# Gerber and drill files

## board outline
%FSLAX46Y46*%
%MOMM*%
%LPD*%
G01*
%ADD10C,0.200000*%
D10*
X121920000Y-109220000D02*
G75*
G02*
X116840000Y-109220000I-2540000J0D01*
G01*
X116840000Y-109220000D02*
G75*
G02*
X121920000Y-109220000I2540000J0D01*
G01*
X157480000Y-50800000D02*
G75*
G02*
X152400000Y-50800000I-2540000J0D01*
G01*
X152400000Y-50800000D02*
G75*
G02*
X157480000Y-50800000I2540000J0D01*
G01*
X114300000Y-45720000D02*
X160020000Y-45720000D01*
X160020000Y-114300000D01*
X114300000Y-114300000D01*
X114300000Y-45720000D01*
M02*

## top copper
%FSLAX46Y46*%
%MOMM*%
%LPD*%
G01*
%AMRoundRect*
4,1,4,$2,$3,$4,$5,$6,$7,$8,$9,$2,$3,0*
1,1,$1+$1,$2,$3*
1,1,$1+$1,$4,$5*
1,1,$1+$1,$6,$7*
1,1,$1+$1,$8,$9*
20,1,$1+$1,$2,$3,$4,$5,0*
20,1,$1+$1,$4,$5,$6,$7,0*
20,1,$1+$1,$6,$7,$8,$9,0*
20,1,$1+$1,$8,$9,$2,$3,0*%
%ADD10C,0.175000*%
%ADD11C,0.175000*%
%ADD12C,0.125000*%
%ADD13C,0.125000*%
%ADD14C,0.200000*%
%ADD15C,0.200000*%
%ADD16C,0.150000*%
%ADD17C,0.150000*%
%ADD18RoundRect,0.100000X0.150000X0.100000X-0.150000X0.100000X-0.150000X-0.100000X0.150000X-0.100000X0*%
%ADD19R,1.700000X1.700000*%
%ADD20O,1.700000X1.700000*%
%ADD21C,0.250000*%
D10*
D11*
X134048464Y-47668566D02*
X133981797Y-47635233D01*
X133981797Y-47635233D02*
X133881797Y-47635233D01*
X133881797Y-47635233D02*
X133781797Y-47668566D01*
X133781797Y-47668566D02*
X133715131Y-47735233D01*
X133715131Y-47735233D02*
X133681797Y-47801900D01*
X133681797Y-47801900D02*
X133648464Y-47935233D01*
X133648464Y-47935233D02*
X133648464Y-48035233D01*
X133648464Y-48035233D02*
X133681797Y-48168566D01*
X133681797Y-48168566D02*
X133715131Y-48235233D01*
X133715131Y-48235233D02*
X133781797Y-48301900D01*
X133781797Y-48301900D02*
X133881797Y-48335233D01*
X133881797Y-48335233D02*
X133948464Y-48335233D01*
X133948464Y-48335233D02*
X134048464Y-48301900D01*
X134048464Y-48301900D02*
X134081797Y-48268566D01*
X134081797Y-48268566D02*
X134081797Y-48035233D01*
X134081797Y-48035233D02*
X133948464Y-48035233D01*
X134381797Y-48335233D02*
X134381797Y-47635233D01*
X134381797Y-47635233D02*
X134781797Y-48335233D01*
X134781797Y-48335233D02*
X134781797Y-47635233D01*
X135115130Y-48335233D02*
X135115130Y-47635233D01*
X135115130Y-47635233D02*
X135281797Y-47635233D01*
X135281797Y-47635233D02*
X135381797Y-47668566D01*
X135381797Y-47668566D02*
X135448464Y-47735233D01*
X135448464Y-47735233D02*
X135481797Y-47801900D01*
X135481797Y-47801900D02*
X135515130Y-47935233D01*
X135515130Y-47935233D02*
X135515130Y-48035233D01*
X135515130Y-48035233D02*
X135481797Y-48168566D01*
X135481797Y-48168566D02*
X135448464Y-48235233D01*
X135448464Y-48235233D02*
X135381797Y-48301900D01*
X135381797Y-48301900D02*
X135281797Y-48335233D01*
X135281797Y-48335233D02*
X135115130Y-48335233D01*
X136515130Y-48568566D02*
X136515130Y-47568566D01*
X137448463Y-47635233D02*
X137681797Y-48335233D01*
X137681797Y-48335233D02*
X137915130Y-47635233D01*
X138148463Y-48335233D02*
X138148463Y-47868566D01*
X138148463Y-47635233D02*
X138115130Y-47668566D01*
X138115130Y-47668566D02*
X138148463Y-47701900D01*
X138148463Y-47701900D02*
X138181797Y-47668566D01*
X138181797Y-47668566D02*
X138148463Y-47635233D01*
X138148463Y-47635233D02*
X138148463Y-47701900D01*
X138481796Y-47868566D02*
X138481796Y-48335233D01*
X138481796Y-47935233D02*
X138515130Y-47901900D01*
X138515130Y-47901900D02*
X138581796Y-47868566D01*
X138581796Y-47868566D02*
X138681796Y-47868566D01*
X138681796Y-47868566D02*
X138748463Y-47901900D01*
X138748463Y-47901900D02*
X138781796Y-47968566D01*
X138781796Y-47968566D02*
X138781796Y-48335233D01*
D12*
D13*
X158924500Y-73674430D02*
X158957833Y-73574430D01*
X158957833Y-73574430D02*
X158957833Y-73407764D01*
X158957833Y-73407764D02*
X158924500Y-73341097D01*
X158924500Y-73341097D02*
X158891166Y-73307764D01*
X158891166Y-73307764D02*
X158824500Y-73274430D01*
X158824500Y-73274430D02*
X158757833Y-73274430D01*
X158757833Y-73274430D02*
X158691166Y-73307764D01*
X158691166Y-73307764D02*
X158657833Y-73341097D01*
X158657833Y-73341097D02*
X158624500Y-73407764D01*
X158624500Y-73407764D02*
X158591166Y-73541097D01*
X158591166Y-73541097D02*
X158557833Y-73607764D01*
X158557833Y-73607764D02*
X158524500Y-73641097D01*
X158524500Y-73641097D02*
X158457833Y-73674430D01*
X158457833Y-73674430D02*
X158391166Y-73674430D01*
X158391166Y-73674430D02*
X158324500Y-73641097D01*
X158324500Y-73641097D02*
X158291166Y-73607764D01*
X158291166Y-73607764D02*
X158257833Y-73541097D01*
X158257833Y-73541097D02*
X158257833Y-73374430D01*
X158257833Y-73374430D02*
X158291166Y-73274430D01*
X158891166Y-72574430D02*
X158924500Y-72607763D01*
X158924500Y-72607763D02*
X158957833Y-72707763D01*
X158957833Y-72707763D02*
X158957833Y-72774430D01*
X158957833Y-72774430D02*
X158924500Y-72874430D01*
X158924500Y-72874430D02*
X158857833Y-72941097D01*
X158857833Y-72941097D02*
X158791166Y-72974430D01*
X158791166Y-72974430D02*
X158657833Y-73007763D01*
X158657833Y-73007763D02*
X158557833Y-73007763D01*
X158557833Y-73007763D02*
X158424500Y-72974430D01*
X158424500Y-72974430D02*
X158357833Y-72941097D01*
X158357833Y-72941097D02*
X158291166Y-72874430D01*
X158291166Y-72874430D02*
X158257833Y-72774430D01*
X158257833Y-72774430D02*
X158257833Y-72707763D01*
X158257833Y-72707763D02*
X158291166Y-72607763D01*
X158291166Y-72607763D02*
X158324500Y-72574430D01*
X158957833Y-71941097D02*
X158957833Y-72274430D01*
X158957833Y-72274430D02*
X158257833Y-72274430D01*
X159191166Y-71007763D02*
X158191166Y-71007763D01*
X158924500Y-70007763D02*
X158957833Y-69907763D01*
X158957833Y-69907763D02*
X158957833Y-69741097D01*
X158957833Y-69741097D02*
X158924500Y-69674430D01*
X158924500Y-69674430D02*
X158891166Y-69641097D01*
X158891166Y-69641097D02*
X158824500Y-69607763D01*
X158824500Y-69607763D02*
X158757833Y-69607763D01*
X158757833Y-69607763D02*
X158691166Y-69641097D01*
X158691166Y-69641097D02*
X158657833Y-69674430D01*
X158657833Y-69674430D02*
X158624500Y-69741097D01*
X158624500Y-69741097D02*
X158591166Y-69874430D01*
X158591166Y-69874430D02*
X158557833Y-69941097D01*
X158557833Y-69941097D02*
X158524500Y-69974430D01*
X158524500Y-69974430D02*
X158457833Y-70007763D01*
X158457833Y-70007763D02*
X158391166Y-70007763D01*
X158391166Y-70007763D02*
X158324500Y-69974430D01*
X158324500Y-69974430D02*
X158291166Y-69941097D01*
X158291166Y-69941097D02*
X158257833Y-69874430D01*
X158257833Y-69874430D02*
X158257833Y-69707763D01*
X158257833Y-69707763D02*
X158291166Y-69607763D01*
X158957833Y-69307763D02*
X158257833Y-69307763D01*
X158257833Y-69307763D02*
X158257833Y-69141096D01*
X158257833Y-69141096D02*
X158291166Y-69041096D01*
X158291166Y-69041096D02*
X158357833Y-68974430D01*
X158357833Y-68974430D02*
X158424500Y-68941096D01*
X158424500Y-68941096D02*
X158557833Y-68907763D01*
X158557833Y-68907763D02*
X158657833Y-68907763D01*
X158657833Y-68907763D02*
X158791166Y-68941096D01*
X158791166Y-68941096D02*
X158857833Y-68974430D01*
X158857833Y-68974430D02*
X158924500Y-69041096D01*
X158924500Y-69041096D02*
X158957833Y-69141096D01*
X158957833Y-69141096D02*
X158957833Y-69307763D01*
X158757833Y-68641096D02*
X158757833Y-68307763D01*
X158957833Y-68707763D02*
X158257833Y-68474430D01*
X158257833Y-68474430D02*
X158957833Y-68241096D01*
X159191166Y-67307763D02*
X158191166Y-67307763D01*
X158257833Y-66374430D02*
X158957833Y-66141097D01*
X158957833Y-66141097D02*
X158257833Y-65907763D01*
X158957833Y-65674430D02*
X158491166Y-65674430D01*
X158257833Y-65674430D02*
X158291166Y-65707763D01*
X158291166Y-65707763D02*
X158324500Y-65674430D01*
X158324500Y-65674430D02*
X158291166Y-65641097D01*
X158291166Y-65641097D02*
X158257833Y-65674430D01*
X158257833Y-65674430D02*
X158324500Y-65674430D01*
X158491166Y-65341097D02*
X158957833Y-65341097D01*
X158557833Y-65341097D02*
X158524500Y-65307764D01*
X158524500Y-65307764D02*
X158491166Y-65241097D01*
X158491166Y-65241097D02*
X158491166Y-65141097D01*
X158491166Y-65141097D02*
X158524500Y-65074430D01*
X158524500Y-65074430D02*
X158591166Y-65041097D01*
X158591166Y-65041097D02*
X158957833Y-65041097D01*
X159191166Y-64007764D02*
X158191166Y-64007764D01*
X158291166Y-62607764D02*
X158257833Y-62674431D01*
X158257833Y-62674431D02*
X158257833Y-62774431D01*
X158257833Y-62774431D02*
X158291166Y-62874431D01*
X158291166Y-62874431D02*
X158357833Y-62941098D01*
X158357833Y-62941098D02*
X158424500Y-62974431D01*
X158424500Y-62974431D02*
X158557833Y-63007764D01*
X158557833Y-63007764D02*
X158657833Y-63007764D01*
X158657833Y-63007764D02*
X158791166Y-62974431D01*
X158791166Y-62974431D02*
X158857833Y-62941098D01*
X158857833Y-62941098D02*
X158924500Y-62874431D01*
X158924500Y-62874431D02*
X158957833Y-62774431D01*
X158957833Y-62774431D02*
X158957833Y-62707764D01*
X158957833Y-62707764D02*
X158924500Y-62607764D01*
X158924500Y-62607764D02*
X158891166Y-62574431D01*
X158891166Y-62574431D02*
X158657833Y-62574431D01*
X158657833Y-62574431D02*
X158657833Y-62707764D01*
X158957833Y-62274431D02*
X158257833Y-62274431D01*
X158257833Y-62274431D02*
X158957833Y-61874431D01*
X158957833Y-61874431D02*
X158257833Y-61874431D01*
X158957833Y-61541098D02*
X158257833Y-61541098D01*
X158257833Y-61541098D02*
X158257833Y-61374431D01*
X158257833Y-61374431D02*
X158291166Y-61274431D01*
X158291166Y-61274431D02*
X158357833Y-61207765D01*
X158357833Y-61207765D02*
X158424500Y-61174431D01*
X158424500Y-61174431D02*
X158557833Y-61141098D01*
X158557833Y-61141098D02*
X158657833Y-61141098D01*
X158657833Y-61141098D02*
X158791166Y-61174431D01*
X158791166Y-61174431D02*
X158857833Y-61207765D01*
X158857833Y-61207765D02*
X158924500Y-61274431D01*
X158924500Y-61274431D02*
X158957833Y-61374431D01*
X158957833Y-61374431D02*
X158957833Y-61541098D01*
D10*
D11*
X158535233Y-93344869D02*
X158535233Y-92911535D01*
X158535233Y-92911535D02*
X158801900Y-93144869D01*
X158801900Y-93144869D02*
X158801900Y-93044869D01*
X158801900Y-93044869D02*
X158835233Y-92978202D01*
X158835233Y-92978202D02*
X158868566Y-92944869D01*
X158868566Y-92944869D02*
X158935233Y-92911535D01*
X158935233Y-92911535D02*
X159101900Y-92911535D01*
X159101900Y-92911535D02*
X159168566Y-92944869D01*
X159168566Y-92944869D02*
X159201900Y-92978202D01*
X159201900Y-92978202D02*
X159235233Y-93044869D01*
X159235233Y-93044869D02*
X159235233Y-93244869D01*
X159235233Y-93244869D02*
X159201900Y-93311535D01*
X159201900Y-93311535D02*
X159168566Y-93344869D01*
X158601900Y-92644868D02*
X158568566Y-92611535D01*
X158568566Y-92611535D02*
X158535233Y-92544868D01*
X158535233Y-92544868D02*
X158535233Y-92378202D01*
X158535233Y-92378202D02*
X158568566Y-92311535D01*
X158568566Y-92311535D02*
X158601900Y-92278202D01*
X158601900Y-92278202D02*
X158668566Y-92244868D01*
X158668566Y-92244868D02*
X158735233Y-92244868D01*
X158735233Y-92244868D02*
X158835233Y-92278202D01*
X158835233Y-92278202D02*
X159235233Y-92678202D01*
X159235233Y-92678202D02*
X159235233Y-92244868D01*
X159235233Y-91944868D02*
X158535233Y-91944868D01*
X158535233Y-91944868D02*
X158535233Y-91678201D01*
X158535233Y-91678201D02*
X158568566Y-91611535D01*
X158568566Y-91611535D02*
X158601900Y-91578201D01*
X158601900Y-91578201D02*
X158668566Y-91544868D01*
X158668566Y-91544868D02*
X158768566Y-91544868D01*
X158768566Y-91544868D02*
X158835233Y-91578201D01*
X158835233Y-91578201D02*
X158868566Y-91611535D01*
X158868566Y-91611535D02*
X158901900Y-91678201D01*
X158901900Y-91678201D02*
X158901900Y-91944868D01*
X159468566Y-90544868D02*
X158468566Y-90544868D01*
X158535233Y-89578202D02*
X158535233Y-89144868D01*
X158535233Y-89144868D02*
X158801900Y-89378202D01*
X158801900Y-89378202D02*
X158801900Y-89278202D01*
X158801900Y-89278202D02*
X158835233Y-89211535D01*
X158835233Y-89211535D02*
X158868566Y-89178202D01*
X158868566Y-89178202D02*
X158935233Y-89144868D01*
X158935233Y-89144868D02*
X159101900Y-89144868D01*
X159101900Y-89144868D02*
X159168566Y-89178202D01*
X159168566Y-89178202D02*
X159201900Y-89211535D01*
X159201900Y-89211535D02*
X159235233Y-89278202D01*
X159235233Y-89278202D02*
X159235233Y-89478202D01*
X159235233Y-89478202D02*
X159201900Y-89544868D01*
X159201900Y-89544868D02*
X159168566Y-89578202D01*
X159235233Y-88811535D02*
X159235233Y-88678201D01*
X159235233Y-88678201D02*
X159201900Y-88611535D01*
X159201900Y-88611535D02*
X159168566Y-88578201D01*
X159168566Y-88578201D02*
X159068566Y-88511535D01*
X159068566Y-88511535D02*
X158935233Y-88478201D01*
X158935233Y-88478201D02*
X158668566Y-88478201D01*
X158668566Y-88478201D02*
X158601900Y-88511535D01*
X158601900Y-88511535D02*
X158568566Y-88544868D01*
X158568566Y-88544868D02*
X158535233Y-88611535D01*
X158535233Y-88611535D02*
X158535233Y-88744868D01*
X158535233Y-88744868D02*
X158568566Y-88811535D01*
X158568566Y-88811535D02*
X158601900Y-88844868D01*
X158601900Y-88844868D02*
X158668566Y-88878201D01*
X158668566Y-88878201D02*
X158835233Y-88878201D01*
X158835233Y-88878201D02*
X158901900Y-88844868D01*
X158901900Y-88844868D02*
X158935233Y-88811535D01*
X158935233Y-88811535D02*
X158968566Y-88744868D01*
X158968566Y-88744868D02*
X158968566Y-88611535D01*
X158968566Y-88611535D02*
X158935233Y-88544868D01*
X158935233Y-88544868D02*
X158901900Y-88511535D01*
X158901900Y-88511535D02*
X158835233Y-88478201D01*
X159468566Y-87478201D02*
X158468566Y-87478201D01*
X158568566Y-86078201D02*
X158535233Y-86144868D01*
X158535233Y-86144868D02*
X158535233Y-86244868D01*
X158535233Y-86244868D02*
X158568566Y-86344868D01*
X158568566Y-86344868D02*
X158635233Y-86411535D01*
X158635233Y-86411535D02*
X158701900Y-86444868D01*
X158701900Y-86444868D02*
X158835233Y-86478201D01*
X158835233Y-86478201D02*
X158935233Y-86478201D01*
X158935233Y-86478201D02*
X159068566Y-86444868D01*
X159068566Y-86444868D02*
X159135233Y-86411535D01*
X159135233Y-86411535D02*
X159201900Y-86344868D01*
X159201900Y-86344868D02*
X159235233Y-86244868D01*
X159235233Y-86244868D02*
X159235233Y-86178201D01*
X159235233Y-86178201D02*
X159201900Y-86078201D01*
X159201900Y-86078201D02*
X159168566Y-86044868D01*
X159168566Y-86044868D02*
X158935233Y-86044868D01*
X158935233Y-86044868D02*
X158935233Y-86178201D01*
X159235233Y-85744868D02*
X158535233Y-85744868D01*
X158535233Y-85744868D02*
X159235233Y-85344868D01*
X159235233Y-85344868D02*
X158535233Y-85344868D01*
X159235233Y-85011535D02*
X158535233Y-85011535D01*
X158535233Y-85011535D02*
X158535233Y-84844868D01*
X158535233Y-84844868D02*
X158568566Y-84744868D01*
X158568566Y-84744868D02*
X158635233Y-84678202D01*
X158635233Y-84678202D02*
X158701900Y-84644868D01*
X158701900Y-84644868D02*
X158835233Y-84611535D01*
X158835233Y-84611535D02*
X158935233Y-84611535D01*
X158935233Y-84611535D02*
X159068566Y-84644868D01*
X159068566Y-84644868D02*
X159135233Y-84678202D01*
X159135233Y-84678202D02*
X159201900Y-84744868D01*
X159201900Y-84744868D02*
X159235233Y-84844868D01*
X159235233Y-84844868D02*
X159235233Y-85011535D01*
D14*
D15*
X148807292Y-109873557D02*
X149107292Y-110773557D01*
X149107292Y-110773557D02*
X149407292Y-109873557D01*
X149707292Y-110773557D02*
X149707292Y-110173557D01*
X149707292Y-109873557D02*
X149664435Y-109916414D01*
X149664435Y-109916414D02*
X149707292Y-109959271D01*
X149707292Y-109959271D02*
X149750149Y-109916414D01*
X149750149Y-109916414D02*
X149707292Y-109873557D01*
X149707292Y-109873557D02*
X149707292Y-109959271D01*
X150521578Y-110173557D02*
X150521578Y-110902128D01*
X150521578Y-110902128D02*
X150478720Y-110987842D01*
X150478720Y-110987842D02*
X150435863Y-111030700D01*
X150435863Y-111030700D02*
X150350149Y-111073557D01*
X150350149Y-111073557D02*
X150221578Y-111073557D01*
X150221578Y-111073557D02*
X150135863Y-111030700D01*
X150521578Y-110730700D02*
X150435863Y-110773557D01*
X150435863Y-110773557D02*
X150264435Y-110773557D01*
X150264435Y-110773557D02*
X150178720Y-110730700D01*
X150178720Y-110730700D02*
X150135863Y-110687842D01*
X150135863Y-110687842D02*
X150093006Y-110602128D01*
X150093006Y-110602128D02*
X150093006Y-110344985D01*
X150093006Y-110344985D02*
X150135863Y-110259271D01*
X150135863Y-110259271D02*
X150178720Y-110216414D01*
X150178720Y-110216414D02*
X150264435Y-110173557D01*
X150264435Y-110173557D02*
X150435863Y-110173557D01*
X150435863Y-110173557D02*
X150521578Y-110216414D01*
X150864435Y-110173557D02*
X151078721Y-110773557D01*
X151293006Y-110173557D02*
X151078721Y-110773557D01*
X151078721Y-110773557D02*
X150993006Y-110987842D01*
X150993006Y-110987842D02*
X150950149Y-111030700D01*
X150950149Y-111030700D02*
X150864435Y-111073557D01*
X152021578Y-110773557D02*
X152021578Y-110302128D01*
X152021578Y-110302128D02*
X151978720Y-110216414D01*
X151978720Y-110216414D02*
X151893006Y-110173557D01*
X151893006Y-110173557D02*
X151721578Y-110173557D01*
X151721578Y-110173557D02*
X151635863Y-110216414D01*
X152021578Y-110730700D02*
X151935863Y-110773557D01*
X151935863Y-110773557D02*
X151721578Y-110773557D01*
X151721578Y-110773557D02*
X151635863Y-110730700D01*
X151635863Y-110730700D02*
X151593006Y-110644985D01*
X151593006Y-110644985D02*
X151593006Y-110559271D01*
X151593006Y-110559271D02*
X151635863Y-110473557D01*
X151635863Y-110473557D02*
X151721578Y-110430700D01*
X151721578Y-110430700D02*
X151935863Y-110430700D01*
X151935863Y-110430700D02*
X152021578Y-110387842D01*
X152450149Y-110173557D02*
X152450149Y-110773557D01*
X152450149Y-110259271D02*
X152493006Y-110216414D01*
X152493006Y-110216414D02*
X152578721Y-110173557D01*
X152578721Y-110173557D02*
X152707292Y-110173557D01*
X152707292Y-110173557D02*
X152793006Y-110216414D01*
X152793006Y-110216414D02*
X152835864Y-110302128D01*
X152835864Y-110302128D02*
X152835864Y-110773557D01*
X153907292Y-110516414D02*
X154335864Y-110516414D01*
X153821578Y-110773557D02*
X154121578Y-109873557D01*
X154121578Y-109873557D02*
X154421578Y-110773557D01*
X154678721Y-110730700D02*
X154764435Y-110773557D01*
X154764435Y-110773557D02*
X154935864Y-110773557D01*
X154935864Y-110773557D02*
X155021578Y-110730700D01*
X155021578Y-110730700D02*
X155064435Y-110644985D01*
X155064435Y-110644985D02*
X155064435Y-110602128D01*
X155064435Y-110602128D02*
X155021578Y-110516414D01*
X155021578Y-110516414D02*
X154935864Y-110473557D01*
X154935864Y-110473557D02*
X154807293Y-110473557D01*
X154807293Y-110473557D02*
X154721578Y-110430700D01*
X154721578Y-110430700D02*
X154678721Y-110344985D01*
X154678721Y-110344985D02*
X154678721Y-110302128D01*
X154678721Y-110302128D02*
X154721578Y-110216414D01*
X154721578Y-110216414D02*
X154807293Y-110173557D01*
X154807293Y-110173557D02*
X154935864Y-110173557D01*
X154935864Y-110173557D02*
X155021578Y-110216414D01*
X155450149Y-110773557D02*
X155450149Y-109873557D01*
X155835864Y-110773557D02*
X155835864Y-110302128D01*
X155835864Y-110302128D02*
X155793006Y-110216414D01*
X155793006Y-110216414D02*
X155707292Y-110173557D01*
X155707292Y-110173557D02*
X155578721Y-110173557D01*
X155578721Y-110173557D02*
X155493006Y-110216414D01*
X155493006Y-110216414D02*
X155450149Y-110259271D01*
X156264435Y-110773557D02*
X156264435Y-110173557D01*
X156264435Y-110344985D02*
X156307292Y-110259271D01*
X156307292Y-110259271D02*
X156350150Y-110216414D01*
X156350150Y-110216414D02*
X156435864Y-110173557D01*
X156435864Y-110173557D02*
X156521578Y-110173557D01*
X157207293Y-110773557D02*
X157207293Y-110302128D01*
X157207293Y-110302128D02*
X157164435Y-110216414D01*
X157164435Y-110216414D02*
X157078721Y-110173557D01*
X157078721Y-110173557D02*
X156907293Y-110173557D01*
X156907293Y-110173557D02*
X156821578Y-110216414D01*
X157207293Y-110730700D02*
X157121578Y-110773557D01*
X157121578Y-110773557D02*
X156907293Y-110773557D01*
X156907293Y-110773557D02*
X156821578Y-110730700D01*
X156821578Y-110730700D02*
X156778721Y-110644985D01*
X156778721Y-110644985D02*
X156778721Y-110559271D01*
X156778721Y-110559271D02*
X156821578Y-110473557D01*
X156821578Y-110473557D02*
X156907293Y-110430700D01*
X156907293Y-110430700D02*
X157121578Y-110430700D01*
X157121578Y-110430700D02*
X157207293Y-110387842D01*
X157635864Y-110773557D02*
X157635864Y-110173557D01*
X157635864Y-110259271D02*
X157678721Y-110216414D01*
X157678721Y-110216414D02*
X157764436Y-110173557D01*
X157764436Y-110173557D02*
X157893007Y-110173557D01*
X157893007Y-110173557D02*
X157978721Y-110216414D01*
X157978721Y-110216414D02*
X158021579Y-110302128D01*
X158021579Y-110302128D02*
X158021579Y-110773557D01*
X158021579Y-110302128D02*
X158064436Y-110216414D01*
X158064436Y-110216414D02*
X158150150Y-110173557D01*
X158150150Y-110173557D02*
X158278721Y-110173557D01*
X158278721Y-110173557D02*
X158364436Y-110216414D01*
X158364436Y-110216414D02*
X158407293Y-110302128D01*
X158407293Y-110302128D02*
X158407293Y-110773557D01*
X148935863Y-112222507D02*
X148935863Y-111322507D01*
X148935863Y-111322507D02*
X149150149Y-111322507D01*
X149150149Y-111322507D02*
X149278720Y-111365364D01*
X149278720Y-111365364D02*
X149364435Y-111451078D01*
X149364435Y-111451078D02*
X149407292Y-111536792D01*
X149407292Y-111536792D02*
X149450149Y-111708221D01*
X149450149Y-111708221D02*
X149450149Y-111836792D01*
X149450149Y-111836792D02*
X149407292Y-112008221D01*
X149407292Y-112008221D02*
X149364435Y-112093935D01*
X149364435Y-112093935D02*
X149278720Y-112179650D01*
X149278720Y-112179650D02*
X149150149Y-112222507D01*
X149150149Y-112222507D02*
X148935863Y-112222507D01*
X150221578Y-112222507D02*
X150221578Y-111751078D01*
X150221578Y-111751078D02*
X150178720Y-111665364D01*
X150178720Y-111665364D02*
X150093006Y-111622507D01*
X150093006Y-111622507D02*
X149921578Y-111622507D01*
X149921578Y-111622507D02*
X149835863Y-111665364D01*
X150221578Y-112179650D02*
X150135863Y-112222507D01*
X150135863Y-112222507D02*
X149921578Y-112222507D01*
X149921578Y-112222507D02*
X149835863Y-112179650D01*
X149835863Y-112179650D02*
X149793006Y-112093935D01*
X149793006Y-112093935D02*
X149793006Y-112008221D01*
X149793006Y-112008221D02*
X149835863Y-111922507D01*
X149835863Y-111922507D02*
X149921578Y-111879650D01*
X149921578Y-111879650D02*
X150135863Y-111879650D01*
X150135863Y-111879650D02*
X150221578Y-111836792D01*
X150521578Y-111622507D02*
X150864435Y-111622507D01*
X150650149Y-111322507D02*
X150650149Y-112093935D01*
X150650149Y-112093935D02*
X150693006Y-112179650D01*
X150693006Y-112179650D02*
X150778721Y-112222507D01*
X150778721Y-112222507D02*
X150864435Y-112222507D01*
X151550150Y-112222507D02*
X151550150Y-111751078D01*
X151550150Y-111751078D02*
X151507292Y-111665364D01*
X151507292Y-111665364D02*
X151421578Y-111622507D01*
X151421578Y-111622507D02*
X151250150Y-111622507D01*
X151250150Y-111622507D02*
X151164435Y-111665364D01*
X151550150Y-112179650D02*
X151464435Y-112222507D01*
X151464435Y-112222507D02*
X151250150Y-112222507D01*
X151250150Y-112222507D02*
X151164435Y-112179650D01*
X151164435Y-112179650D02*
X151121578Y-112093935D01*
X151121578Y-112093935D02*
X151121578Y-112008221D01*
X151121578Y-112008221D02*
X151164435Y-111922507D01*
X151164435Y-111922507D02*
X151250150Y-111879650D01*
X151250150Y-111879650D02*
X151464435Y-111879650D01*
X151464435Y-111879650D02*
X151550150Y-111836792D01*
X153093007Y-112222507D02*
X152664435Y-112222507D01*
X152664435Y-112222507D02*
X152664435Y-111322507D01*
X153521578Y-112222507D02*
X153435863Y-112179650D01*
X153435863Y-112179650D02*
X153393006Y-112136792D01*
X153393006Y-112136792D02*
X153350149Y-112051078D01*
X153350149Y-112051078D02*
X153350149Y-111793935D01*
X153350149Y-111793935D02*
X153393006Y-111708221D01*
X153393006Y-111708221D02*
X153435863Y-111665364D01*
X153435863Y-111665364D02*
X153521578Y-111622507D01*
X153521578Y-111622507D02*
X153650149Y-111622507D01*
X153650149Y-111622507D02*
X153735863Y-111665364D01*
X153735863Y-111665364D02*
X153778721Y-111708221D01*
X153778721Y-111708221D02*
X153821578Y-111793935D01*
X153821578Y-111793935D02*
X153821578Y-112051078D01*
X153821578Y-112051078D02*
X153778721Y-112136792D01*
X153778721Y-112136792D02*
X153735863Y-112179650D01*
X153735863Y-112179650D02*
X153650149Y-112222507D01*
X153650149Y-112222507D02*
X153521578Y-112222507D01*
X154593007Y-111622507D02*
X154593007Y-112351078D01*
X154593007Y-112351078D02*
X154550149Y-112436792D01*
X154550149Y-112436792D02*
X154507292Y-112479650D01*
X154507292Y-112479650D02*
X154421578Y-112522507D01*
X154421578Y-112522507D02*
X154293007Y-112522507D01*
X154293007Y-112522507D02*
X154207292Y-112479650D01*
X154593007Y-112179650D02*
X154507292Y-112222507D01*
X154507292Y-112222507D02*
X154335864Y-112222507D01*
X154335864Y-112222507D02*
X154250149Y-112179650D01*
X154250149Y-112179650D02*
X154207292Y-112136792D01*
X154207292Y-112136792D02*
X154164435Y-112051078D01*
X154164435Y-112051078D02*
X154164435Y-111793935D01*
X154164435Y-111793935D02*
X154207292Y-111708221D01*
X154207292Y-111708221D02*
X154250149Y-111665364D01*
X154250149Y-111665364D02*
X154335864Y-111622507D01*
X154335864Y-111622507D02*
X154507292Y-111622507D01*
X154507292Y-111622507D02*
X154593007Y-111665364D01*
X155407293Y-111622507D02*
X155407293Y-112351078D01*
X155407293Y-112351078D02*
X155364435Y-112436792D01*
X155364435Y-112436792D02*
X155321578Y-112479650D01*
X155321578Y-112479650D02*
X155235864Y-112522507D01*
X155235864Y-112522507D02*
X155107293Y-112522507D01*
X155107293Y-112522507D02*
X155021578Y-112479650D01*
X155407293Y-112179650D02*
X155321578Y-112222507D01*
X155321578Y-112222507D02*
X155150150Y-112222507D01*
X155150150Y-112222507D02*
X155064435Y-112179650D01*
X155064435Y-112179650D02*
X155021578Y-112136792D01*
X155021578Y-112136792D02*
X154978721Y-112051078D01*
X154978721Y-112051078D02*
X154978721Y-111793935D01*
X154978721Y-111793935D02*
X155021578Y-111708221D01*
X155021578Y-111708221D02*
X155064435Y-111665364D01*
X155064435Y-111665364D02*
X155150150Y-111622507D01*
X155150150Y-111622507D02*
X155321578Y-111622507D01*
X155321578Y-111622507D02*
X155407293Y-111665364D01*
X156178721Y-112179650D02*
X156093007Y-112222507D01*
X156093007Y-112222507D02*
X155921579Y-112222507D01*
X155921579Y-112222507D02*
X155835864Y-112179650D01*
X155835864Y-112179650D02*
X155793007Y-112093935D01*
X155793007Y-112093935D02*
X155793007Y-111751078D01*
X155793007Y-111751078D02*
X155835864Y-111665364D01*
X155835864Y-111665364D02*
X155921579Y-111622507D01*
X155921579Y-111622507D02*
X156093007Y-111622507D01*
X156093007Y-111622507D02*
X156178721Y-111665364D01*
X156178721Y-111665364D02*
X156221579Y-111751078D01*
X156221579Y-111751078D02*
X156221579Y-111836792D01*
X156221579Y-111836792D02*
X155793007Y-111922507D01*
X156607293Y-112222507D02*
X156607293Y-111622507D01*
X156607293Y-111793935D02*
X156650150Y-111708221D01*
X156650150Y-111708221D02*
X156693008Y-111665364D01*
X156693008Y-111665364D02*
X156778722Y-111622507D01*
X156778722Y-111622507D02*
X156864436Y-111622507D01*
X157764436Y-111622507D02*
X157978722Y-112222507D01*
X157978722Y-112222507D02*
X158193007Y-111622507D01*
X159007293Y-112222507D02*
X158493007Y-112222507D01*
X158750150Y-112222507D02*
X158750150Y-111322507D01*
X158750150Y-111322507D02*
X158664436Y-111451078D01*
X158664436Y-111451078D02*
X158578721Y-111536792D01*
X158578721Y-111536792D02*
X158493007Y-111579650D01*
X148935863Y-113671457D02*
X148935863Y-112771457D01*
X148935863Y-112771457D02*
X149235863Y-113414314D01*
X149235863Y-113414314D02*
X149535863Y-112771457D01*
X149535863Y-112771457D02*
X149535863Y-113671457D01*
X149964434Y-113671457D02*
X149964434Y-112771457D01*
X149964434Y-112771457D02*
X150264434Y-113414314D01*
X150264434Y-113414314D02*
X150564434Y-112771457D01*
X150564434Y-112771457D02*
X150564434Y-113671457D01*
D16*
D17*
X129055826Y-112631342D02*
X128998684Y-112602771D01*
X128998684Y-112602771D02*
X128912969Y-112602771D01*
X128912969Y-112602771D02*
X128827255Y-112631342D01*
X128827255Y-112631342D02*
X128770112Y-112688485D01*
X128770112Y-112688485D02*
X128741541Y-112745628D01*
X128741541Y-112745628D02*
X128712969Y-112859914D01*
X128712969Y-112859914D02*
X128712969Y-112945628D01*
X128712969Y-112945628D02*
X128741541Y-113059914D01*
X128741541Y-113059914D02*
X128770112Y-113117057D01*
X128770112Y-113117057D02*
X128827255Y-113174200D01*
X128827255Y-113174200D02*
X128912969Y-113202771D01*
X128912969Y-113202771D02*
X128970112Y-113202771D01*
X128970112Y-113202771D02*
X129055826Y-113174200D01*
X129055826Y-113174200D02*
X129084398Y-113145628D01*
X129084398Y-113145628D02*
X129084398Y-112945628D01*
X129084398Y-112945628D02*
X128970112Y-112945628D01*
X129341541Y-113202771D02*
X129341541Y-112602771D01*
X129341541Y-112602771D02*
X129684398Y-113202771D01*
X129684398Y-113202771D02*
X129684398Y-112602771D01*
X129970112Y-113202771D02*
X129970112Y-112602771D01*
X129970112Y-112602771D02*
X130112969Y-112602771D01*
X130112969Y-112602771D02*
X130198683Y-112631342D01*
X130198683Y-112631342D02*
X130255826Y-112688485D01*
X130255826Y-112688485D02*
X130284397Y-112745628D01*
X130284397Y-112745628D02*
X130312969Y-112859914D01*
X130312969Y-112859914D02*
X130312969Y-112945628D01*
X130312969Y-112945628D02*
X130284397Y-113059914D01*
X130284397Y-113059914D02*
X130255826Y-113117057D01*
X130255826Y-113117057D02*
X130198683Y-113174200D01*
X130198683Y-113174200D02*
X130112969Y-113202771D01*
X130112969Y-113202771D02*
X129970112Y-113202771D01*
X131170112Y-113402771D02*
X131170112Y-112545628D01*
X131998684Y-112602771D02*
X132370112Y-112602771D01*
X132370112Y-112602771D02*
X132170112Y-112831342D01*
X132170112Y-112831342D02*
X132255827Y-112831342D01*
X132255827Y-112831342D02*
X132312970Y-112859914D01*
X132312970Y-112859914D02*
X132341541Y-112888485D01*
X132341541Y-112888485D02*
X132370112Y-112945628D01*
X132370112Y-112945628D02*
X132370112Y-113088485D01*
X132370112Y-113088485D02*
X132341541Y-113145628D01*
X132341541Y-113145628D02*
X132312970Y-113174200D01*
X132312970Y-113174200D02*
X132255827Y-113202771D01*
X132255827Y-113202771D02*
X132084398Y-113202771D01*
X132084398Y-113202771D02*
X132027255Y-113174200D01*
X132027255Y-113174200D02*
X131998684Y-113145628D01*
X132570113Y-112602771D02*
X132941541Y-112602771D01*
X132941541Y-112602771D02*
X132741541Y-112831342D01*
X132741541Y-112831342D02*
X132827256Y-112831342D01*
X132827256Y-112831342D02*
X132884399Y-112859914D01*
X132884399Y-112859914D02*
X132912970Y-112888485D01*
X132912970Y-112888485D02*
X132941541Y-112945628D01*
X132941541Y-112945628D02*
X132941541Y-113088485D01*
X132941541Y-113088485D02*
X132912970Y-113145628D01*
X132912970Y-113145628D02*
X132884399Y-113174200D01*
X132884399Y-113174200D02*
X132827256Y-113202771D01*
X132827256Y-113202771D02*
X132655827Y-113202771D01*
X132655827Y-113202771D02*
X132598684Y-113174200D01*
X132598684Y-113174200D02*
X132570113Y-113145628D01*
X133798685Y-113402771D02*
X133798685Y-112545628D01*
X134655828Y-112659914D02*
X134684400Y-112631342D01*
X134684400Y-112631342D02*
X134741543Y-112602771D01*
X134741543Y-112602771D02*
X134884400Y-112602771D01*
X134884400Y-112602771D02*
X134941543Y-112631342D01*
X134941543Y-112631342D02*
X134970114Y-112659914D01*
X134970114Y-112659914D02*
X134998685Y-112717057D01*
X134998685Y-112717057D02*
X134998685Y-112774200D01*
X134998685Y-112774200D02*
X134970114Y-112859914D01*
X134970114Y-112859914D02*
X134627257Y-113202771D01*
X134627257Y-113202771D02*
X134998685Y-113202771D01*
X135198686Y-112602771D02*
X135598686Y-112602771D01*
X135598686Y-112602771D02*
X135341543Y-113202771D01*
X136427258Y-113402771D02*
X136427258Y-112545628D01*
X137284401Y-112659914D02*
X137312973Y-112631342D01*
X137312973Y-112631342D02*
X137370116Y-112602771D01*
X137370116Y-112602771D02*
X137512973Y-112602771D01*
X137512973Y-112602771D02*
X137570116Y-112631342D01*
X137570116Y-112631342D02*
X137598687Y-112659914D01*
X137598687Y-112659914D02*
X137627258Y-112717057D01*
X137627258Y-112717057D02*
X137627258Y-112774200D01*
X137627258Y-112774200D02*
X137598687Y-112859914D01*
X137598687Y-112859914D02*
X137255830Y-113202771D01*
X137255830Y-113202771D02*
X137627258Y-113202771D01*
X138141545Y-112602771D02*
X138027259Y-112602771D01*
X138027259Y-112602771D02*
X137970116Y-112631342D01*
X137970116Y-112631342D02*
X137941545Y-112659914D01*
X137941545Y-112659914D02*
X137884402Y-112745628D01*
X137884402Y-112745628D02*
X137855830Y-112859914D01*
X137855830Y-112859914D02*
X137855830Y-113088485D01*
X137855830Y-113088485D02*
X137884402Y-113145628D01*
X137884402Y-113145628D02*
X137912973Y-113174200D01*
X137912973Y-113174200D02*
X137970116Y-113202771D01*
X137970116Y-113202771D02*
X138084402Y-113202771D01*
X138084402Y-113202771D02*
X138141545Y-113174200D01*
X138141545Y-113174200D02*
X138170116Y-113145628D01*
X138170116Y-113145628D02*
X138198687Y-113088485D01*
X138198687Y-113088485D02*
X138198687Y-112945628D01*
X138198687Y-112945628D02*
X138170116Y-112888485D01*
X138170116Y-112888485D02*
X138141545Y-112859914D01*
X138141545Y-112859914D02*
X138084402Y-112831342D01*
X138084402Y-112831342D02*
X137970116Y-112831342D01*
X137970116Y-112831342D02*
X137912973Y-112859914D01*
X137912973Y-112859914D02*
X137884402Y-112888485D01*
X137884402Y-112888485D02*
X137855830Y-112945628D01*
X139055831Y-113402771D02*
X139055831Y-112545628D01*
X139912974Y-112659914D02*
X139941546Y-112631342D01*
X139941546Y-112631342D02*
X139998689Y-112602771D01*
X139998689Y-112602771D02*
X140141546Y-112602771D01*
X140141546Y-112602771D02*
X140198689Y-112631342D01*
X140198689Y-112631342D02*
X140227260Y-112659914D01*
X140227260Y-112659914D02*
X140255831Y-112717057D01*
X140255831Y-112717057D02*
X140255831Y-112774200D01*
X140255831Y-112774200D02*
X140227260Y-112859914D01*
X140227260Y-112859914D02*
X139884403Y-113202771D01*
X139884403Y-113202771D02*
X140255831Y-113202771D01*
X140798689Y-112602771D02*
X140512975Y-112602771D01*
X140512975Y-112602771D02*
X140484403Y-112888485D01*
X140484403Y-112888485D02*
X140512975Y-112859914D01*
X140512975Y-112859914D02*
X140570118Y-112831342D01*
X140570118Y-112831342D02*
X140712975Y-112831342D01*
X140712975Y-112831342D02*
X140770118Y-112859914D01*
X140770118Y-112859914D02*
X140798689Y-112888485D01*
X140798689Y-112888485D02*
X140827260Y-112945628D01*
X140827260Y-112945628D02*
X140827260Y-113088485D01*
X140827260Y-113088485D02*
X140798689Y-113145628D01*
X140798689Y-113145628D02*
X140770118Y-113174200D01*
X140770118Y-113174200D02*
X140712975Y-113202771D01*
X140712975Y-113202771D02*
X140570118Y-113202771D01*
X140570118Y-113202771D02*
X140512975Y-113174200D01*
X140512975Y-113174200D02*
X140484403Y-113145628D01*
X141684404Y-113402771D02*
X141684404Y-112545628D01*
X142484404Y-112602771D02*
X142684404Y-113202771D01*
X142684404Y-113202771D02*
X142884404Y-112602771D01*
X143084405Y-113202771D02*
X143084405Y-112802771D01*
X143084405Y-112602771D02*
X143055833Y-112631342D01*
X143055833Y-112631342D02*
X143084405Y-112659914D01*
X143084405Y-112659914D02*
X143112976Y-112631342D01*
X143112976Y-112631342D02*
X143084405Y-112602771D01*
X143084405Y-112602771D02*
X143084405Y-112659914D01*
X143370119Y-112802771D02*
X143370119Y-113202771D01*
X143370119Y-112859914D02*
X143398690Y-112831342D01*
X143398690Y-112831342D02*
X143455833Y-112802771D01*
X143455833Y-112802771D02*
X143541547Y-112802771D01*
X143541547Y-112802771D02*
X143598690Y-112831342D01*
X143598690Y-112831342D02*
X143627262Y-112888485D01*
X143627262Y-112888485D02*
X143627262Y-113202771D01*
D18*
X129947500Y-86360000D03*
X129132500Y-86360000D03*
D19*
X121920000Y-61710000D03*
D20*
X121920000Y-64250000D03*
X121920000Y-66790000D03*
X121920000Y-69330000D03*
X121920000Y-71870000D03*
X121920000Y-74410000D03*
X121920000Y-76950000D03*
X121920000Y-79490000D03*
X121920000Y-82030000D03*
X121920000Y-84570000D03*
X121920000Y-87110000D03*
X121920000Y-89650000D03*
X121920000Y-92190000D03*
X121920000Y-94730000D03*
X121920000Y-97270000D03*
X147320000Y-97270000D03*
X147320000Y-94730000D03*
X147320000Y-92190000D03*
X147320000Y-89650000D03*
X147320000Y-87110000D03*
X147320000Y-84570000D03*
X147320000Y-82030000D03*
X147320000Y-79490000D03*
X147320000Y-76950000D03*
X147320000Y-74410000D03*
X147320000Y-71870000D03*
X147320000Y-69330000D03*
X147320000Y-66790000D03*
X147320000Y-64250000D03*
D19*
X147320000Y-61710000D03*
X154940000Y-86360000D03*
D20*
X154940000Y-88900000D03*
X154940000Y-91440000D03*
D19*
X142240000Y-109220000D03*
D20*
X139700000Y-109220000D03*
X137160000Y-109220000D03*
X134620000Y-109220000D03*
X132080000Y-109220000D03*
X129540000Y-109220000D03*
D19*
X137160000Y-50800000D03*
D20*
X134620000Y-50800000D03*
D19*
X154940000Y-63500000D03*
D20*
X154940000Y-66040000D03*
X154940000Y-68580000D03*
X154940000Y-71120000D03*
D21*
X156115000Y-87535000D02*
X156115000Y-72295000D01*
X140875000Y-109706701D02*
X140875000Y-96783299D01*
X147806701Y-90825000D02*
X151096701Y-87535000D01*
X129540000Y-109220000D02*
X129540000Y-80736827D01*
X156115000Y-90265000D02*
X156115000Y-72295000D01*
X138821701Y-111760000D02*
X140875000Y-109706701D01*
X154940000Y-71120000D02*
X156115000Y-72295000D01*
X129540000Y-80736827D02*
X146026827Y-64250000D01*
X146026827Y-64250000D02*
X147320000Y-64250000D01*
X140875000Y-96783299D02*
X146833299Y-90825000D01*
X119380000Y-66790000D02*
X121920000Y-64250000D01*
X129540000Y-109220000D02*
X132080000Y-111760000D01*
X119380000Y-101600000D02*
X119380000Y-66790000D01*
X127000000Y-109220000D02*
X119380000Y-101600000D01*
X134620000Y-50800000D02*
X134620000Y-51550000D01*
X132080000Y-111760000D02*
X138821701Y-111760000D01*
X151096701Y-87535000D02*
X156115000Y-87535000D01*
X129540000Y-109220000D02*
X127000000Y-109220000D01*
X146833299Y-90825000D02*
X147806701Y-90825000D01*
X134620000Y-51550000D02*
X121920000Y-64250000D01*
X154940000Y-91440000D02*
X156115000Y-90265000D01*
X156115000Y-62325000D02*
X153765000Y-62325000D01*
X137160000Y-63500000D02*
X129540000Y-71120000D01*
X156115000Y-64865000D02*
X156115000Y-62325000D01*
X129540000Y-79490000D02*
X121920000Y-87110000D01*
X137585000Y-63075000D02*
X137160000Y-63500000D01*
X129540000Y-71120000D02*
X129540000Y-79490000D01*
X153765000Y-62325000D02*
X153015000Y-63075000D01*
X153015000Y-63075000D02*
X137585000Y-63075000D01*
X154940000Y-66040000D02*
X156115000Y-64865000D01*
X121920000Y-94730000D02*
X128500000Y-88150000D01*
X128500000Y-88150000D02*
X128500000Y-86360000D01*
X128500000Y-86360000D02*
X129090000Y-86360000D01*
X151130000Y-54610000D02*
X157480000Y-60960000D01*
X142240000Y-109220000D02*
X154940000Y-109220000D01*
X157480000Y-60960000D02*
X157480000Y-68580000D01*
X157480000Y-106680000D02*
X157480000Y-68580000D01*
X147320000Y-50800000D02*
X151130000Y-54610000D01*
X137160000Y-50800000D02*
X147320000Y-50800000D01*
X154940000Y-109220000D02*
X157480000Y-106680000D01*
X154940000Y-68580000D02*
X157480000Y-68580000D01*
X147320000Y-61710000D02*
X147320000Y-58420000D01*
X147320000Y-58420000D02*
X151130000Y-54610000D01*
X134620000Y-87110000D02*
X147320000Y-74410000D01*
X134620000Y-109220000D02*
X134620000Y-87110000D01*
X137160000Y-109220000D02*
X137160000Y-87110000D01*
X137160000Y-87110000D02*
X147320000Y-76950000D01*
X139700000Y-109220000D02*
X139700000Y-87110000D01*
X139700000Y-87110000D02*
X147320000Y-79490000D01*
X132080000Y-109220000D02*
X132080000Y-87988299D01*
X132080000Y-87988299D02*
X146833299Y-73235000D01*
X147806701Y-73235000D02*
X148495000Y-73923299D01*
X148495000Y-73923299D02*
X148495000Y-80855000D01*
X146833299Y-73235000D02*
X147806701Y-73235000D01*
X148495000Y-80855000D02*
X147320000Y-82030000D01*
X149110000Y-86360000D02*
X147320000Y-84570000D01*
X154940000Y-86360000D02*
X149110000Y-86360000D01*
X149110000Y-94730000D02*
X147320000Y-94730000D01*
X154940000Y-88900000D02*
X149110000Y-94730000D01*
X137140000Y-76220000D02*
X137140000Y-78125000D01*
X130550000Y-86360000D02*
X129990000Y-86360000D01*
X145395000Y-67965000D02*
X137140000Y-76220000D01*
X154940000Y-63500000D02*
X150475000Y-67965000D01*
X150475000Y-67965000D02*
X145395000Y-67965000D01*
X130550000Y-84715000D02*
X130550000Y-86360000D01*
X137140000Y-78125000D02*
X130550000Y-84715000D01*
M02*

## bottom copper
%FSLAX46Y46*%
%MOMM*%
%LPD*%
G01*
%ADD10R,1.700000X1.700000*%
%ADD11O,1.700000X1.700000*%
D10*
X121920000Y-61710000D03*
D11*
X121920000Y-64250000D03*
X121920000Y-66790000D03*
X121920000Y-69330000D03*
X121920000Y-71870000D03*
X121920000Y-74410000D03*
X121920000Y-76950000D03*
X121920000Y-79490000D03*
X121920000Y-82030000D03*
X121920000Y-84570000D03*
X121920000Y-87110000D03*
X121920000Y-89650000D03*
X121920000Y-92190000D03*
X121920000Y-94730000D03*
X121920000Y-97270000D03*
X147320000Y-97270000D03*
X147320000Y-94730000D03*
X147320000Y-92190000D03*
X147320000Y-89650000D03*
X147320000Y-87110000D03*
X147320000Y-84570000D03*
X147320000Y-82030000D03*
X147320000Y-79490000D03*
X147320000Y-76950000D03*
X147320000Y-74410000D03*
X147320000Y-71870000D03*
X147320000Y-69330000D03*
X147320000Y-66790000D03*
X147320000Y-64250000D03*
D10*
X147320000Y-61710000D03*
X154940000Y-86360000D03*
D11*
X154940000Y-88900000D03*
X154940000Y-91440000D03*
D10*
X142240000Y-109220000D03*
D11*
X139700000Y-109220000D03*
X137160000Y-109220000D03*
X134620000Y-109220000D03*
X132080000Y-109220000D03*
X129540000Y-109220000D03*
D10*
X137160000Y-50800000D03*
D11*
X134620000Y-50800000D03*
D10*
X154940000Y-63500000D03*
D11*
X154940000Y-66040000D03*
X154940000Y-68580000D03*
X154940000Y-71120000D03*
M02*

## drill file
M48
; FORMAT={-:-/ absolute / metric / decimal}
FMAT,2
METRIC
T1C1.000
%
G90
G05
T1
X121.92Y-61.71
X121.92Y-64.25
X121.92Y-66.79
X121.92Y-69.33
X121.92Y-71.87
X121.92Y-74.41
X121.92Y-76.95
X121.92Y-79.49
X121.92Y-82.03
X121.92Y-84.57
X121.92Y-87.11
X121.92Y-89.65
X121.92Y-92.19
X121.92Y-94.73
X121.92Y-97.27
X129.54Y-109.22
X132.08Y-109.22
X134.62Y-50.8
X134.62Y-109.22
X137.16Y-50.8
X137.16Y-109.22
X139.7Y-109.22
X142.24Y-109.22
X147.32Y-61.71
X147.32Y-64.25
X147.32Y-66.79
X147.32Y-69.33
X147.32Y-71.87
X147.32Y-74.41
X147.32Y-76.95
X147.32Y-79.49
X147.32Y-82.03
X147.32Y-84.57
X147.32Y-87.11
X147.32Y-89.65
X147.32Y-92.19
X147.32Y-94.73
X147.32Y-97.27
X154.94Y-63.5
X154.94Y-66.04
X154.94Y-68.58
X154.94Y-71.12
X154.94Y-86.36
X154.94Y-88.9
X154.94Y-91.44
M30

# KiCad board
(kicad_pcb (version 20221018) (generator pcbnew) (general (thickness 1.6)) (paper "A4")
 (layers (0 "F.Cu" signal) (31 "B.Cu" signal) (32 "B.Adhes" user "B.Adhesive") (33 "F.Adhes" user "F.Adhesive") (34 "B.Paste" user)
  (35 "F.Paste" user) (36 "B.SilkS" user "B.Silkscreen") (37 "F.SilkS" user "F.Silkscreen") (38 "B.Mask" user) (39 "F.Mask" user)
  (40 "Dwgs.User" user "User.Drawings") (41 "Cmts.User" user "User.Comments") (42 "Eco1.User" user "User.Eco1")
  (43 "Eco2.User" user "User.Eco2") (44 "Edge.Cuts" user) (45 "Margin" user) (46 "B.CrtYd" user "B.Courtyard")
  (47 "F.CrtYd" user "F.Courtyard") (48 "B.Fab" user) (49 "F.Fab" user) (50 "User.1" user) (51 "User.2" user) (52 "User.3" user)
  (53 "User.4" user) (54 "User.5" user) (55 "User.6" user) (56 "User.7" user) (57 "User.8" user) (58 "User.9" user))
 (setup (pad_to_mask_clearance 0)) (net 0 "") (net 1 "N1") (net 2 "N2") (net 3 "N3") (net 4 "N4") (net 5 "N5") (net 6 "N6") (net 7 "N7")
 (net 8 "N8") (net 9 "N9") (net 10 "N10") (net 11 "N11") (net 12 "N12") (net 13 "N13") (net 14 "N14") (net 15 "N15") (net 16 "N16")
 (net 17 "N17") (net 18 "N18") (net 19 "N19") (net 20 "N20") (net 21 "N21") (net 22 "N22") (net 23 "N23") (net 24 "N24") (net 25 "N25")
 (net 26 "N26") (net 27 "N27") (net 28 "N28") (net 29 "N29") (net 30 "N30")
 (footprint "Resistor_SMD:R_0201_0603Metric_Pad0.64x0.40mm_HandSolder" (layer "F.Cu") (at 129.54 86.36 180)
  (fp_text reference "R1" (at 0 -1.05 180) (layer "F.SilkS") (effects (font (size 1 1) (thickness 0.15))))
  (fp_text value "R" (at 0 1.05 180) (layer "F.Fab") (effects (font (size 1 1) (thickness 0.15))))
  (pad "" smd roundrect (at -0.46 0 180) (size 0.4 0.36) (layers "F.Paste") (roundrect_rratio 0.25))
  (pad "" smd roundrect (at 0.4325 0 180) (size 0.458 0.36) (layers "F.Paste") (roundrect_rratio 0.25))
  (pad "1" smd roundrect (at -0.4075 0 180) (size 0.5 0.4) (layers "F.Cu" "F.Mask") (roundrect_rratio 0.25) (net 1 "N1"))
  (pad "2" smd roundrect (at 0.4075 0 180) (size 0.5 0.4) (layers "F.Cu" "F.Mask") (roundrect_rratio 0.25) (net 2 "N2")))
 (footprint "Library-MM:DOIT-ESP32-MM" (layer "F.Cu") (at 121.92 60.96)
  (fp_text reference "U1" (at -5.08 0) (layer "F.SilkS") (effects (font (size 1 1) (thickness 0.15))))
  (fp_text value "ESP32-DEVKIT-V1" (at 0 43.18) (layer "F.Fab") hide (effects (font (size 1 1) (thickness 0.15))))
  (pad "1" thru_hole rect (at 0 0.75) (size 1.7 1.7) (drill 1) (layers "*.Cu" "*.Mask") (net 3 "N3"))
  (pad "2" thru_hole oval (at 0 3.29) (size 1.7 1.7) (drill 1) (layers "*.Cu" "*.Mask") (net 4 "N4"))
  (pad "3" thru_hole oval (at 0 5.83) (size 1.7 1.7) (drill 1) (layers "*.Cu" "*.Mask") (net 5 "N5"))
  (pad "4" thru_hole oval (at 0 8.37) (size 1.7 1.7) (drill 1) (layers "*.Cu" "*.Mask") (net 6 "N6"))
  (pad "5" thru_hole oval (at 0 10.91) (size 1.7 1.7) (drill 1) (layers "*.Cu" "*.Mask") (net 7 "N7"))
  (pad "6" thru_hole oval (at 0 13.45) (size 1.7 1.7) (drill 1) (layers "*.Cu" "*.Mask") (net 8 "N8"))
  (pad "7" thru_hole oval (at 0 15.99) (size 1.7 1.7) (drill 1) (layers "*.Cu" "*.Mask") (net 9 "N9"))
  (pad "8" thru_hole oval (at 0 18.53) (size 1.7 1.7) (drill 1) (layers "*.Cu" "*.Mask") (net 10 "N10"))
  (pad "9" thru_hole oval (at 0 21.07) (size 1.7 1.7) (drill 1) (layers "*.Cu" "*.Mask") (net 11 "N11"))
  (pad "10" thru_hole oval (at 0 23.61) (size 1.7 1.7) (drill 1) (layers "*.Cu" "*.Mask") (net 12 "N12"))
  (pad "11" thru_hole oval (at 0 26.15) (size 1.7 1.7) (drill 1) (layers "*.Cu" "*.Mask") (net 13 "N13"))
  (pad "12" thru_hole oval (at 0 28.69) (size 1.7 1.7) (drill 1) (layers "*.Cu" "*.Mask") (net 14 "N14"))
  (pad "13" thru_hole oval (at 0 31.23) (size 1.7 1.7) (drill 1) (layers "*.Cu" "*.Mask") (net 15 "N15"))
  (pad "14" thru_hole oval (at 0 33.77) (size 1.7 1.7) (drill 1) (layers "*.Cu" "*.Mask") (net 2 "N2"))
  (pad "15" thru_hole oval (at 0 36.31) (size 1.7 1.7) (drill 1) (layers "*.Cu" "*.Mask") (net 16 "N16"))
  (pad "16" thru_hole oval (at 25.4 36.31) (size 1.7 1.7) (drill 1) (layers "*.Cu" "*.Mask") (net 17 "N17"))
  (pad "17" thru_hole oval (at 25.4 33.77) (size 1.7 1.7) (drill 1) (layers "*.Cu" "*.Mask") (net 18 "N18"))
  (pad "18" thru_hole oval (at 25.4 31.23) (size 1.7 1.7) (drill 1) (layers "*.Cu" "*.Mask") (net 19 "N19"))
  (pad "19" thru_hole oval (at 25.4 28.69) (size 1.7 1.7) (drill 1) (layers "*.Cu" "*.Mask") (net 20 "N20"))
  (pad "20" thru_hole oval (at 25.4 26.15) (size 1.7 1.7) (drill 1) (layers "*.Cu" "*.Mask") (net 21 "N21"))
  (pad "21" thru_hole oval (at 25.4 23.61) (size 1.7 1.7) (drill 1) (layers "*.Cu" "*.Mask") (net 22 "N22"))
  (pad "22" thru_hole oval (at 25.4 21.07) (size 1.7 1.7) (drill 1) (layers "*.Cu" "*.Mask") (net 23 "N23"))
  (pad "23" thru_hole oval (at 25.4 18.53) (size 1.7 1.7) (drill 1) (layers "*.Cu" "*.Mask") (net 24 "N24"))
  (pad "24" thru_hole oval (at 25.4 15.99) (size 1.7 1.7) (drill 1) (layers "*.Cu" "*.Mask") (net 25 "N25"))
  (pad "25" thru_hole oval (at 25.4 13.45) (size 1.7 1.7) (drill 1) (layers "*.Cu" "*.Mask") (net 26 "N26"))
  (pad "26" thru_hole oval (at 25.4 10.91) (size 1.7 1.7) (drill 1) (layers "*.Cu" "*.Mask") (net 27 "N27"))
  (pad "27" thru_hole oval (at 25.4 8.37) (size 1.7 1.7) (drill 1) (layers "*.Cu" "*.Mask") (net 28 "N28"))
  (pad "28" thru_hole oval (at 25.4 5.83) (size 1.7 1.7) (drill 1) (layers "*.Cu" "*.Mask") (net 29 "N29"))
  (pad "29" thru_hole oval (at 25.4 3.29) (size 1.7 1.7) (drill 1) (layers "*.Cu" "*.Mask") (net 4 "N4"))
  (pad "30" thru_hole rect (at 25.4 0.75) (size 1.7 1.7) (drill 1) (layers "*.Cu" "*.Mask") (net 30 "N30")))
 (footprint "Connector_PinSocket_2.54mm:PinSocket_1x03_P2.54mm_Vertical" (layer "F.Cu") (at 154.94 86.36)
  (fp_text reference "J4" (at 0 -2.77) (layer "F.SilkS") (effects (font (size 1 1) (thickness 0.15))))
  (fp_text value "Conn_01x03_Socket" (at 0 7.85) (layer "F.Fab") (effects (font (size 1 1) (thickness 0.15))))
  (pad "1" thru_hole rect (at 0 0) (size 1.7 1.7) (drill 1) (layers "*.Cu" "*.Mask") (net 22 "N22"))
  (pad "2" thru_hole oval (at 0 2.54) (size 1.7 1.7) (drill 1) (layers "*.Cu" "*.Mask") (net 18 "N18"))
  (pad "3" thru_hole oval (at 0 5.08) (size 1.7 1.7) (drill 1) (layers "*.Cu" "*.Mask") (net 4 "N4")))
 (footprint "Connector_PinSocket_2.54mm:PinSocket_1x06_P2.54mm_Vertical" (layer "F.Cu") (at 142.24 109.22 -90)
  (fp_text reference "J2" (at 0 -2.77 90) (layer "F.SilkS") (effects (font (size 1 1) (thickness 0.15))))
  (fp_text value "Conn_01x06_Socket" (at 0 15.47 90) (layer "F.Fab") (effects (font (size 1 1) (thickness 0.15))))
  (pad "1" thru_hole rect (at 0 0 270) (size 1.7 1.7) (drill 1) (layers "*.Cu" "*.Mask") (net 30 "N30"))
  (pad "2" thru_hole oval (at 0 2.54 270) (size 1.7 1.7) (drill 1) (layers "*.Cu" "*.Mask") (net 24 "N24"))
  (pad "3" thru_hole oval (at 0 5.08 270) (size 1.7 1.7) (drill 1) (layers "*.Cu" "*.Mask") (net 25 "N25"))
  (pad "4" thru_hole oval (at 0 7.62 270) (size 1.7 1.7) (drill 1) (layers "*.Cu" "*.Mask") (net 26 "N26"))
  (pad "5" thru_hole oval (at 0 10.16 270) (size 1.7 1.7) (drill 1) (layers "*.Cu" "*.Mask") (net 23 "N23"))
  (pad "6" thru_hole oval (at 0 12.7 270) (size 1.7 1.7) (drill 1) (layers "*.Cu" "*.Mask") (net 4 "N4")))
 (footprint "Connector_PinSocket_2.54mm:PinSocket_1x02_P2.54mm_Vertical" (layer "F.Cu") (at 137.16 50.8 -90)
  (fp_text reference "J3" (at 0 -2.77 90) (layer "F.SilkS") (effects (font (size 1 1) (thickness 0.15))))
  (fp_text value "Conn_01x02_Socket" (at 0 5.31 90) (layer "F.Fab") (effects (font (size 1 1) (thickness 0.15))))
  (pad "1" thru_hole rect (at 0 0 270) (size 1.7 1.7) (drill 1) (layers "*.Cu" "*.Mask") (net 30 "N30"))
  (pad "2" thru_hole oval (at 0 2.54 270) (size 1.7 1.7) (drill 1) (layers "*.Cu" "*.Mask") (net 4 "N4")))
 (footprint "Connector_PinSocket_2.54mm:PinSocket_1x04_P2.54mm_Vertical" (layer "F.Cu") (at 154.94 63.5)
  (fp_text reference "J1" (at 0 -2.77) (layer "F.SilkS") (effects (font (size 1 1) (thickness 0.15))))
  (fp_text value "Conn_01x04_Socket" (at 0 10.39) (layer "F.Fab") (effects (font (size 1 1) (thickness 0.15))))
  (pad "1" thru_hole rect (at 0 0) (size 1.7 1.7) (drill 1) (layers "*.Cu" "*.Mask") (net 1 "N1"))
  (pad "2" thru_hole oval (at 0 2.54) (size 1.7 1.7) (drill 1) (layers "*.Cu" "*.Mask") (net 13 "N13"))
  (pad "3" thru_hole oval (at 0 5.08) (size 1.7 1.7) (drill 1) (layers "*.Cu" "*.Mask") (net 30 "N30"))
  (pad "4" thru_hole oval (at 0 7.62) (size 1.7 1.7) (drill 1) (layers "*.Cu" "*.Mask") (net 4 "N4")))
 (gr_circle (center 119.38 109.22) (end 121.92 109.22) (stroke (width 0.2) (type default)) (fill none) (layer "Edge.Cuts"))
 (gr_circle (center 154.94 50.8) (end 157.48 50.8) (stroke (width 0.2) (type solid)) (fill none) (layer "Edge.Cuts"))
 (gr_rect (start 114.3 45.72) (end 160.02 114.3) (stroke (width 0.2) (type default)) (fill none) (layer "Edge.Cuts"))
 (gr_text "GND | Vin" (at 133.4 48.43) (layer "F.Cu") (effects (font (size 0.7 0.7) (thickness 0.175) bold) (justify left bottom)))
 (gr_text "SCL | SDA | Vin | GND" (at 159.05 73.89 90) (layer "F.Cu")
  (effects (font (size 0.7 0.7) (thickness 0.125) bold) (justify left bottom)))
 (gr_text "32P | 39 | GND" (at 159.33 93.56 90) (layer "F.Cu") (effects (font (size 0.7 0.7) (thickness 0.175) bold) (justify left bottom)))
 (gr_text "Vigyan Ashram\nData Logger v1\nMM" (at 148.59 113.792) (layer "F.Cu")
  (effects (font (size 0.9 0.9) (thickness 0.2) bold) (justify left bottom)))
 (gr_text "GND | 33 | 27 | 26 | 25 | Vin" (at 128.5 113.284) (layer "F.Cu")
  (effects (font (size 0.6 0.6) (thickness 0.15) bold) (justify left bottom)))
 (segment (start 156.115 87.535) (end 156.115 72.295) (width 0.25) (layer "F.Cu") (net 4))
 (segment (start 140.875 109.706701) (end 140.875 96.783299) (width 0.25) (layer "F.Cu") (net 4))
 (segment (start 147.806701 90.825) (end 151.096701 87.535) (width 0.25) (layer "F.Cu") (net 4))
 (segment (start 129.54 109.22) (end 129.54 80.736827) (width 0.25) (layer "F.Cu") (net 4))
 (segment (start 156.115 90.265) (end 156.115 72.295) (width 0.25) (layer "F.Cu") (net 4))
 (segment (start 138.821701 111.76) (end 140.875 109.706701) (width 0.25) (layer "F.Cu") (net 4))
 (segment (start 154.94 71.12) (end 156.115 72.295) (width 0.25) (layer "F.Cu") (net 4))
 (segment (start 129.54 80.736827) (end 146.026827 64.25) (width 0.25) (layer "F.Cu") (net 4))
 (segment (start 146.026827 64.25) (end 147.32 64.25) (width 0.25) (layer "F.Cu") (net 4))
 (segment (start 140.875 96.783299) (end 146.833299 90.825) (width 0.25) (layer "F.Cu") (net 4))
 (segment (start 119.38 66.79) (end 121.92 64.25) (width 0.25) (layer "F.Cu") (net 4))
 (segment (start 129.54 109.22) (end 132.08 111.76) (width 0.25) (layer "F.Cu") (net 4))
 (segment (start 119.38 101.6) (end 119.38 66.79) (width 0.25) (layer "F.Cu") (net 4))
 (segment (start 127 109.22) (end 119.38 101.6) (width 0.25) (layer "F.Cu") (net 4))
 (segment (start 134.62 50.8) (end 134.62 51.55) (width 0.25) (layer "F.Cu") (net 4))
 (segment (start 132.08 111.76) (end 138.821701 111.76) (width 0.25) (layer "F.Cu") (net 4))
 (segment (start 151.096701 87.535) (end 156.115 87.535) (width 0.25) (layer "F.Cu") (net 4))
 (segment (start 129.54 109.22) (end 127 109.22) (width 0.25) (layer "F.Cu") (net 4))
 (segment (start 146.833299 90.825) (end 147.806701 90.825) (width 0.25) (layer "F.Cu") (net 4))
 (segment (start 134.62 51.55) (end 121.92 64.25) (width 0.25) (layer "F.Cu") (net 4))
 (segment (start 154.94 91.44) (end 156.115 90.265) (width 0.25) (layer "F.Cu") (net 4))
 (segment (start 156.115 62.325) (end 153.765 62.325) (width 0.25) (layer "F.Cu") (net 13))
 (segment (start 137.16 63.5) (end 129.54 71.12) (width 0.25) (layer "F.Cu") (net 13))
 (segment (start 156.115 64.865) (end 156.115 62.325) (width 0.25) (layer "F.Cu") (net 13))
 (segment (start 129.54 79.49) (end 121.92 87.11) (width 0.25) (layer "F.Cu") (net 13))
 (segment (start 137.585 63.075) (end 137.16 63.5) (width 0.25) (layer "F.Cu") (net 13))
 (segment (start 129.54 71.12) (end 129.54 79.49) (width 0.25) (layer "F.Cu") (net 13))
 (segment (start 153.765 62.325) (end 153.015 63.075) (width 0.25) (layer "F.Cu") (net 13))
 (segment (start 153.015 63.075) (end 137.585 63.075) (width 0.25) (layer "F.Cu") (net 13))
 (segment (start 154.94 66.04) (end 156.115 64.865) (width 0.25) (layer "F.Cu") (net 13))
 (segment (start 121.92 94.73) (end 128.5 88.15) (width 0.25) (layer "F.Cu") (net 2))
 (segment (start 128.5 88.15) (end 128.5 86.36) (width 0.25) (layer "F.Cu") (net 2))
 (segment (start 128.5 86.36) (end 129.09 86.36) (width 0.25) (layer "F.Cu") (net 2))
 (segment (start 151.13 54.61) (end 157.48 60.96) (width 0.25) (layer "F.Cu") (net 30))
 (segment (start 142.24 109.22) (end 154.94 109.22) (width 0.25) (layer "F.Cu") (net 30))
 (segment (start 157.48 60.96) (end 157.48 68.58) (width 0.25) (layer "F.Cu") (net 30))
 (segment (start 157.48 106.68) (end 157.48 68.58) (width 0.25) (layer "F.Cu") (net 30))
 (segment (start 147.32 50.8) (end 151.13 54.61) (width 0.25) (layer "F.Cu") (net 30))
 (segment (start 137.16 50.8) (end 147.32 50.8) (width 0.25) (layer "F.Cu") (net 30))
 (segment (start 154.94 109.22) (end 157.48 106.68) (width 0.25) (layer "F.Cu") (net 30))
 (segment (start 154.94 68.58) (end 157.48 68.58) (width 0.25) (layer "F.Cu") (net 30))
 (segment (start 147.32 61.71) (end 147.32 58.42) (width 0.25) (layer "F.Cu") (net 30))
 (segment (start 147.32 58.42) (end 151.13 54.61) (width 0.25) (layer "F.Cu") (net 30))
 (segment (start 134.62 87.11) (end 147.32 74.41) (width 0.25) (layer "F.Cu") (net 26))
 (segment (start 134.62 109.22) (end 134.62 87.11) (width 0.25) (layer "F.Cu") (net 26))
 (segment (start 137.16 109.22) (end 137.16 87.11) (width 0.25) (layer "F.Cu") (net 25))
 (segment (start 137.16 87.11) (end 147.32 76.95) (width 0.25) (layer "F.Cu") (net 25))
 (segment (start 139.7 109.22) (end 139.7 87.11) (width 0.25) (layer "F.Cu") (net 24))
 (segment (start 139.7 87.11) (end 147.32 79.49) (width 0.25) (layer "F.Cu") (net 24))
 (segment (start 132.08 109.22) (end 132.08 87.988299) (width 0.25) (layer "F.Cu") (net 23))
 (segment (start 132.08 87.988299) (end 146.833299 73.235) (width 0.25) (layer "F.Cu") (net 23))
 (segment (start 147.806701 73.235) (end 148.495 73.923299) (width 0.25) (layer "F.Cu") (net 23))
 (segment (start 148.495 73.923299) (end 148.495 80.855) (width 0.25) (layer "F.Cu") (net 23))
 (segment (start 146.833299 73.235) (end 147.806701 73.235) (width 0.25) (layer "F.Cu") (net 23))
 (segment (start 148.495 80.855) (end 147.32 82.03) (width 0.25) (layer "F.Cu") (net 23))
 (segment (start 149.11 86.36) (end 147.32 84.57) (width 0.25) (layer "F.Cu") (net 22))
 (segment (start 154.94 86.36) (end 149.11 86.36) (width 0.25) (layer "F.Cu") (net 22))
 (segment (start 149.11 94.73) (end 147.32 94.73) (width 0.25) (layer "F.Cu") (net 18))
 (segment (start 154.94 88.9) (end 149.11 94.73) (width 0.25) (layer "F.Cu") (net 18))
 (segment (start 137.14 76.22) (end 137.14 78.125) (width 0.25) (layer "F.Cu") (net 1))
 (segment (start 130.55 86.36) (end 129.99 86.36) (width 0.25) (layer "F.Cu") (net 1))
 (segment (start 145.395 67.965) (end 137.14 76.22) (width 0.25) (layer "F.Cu") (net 1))
 (segment (start 154.94 63.5) (end 150.475 67.965) (width 0.25) (layer "F.Cu") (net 1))
 (segment (start 150.475 67.965) (end 145.395 67.965) (width 0.25) (layer "F.Cu") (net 1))
 (segment (start 130.55 84.715) (end 130.55 86.36) (width 0.25) (layer "F.Cu") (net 1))
 (segment (start 137.14 78.125) (end 130.55 84.715) (width 0.25) (layer "F.Cu") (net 1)))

